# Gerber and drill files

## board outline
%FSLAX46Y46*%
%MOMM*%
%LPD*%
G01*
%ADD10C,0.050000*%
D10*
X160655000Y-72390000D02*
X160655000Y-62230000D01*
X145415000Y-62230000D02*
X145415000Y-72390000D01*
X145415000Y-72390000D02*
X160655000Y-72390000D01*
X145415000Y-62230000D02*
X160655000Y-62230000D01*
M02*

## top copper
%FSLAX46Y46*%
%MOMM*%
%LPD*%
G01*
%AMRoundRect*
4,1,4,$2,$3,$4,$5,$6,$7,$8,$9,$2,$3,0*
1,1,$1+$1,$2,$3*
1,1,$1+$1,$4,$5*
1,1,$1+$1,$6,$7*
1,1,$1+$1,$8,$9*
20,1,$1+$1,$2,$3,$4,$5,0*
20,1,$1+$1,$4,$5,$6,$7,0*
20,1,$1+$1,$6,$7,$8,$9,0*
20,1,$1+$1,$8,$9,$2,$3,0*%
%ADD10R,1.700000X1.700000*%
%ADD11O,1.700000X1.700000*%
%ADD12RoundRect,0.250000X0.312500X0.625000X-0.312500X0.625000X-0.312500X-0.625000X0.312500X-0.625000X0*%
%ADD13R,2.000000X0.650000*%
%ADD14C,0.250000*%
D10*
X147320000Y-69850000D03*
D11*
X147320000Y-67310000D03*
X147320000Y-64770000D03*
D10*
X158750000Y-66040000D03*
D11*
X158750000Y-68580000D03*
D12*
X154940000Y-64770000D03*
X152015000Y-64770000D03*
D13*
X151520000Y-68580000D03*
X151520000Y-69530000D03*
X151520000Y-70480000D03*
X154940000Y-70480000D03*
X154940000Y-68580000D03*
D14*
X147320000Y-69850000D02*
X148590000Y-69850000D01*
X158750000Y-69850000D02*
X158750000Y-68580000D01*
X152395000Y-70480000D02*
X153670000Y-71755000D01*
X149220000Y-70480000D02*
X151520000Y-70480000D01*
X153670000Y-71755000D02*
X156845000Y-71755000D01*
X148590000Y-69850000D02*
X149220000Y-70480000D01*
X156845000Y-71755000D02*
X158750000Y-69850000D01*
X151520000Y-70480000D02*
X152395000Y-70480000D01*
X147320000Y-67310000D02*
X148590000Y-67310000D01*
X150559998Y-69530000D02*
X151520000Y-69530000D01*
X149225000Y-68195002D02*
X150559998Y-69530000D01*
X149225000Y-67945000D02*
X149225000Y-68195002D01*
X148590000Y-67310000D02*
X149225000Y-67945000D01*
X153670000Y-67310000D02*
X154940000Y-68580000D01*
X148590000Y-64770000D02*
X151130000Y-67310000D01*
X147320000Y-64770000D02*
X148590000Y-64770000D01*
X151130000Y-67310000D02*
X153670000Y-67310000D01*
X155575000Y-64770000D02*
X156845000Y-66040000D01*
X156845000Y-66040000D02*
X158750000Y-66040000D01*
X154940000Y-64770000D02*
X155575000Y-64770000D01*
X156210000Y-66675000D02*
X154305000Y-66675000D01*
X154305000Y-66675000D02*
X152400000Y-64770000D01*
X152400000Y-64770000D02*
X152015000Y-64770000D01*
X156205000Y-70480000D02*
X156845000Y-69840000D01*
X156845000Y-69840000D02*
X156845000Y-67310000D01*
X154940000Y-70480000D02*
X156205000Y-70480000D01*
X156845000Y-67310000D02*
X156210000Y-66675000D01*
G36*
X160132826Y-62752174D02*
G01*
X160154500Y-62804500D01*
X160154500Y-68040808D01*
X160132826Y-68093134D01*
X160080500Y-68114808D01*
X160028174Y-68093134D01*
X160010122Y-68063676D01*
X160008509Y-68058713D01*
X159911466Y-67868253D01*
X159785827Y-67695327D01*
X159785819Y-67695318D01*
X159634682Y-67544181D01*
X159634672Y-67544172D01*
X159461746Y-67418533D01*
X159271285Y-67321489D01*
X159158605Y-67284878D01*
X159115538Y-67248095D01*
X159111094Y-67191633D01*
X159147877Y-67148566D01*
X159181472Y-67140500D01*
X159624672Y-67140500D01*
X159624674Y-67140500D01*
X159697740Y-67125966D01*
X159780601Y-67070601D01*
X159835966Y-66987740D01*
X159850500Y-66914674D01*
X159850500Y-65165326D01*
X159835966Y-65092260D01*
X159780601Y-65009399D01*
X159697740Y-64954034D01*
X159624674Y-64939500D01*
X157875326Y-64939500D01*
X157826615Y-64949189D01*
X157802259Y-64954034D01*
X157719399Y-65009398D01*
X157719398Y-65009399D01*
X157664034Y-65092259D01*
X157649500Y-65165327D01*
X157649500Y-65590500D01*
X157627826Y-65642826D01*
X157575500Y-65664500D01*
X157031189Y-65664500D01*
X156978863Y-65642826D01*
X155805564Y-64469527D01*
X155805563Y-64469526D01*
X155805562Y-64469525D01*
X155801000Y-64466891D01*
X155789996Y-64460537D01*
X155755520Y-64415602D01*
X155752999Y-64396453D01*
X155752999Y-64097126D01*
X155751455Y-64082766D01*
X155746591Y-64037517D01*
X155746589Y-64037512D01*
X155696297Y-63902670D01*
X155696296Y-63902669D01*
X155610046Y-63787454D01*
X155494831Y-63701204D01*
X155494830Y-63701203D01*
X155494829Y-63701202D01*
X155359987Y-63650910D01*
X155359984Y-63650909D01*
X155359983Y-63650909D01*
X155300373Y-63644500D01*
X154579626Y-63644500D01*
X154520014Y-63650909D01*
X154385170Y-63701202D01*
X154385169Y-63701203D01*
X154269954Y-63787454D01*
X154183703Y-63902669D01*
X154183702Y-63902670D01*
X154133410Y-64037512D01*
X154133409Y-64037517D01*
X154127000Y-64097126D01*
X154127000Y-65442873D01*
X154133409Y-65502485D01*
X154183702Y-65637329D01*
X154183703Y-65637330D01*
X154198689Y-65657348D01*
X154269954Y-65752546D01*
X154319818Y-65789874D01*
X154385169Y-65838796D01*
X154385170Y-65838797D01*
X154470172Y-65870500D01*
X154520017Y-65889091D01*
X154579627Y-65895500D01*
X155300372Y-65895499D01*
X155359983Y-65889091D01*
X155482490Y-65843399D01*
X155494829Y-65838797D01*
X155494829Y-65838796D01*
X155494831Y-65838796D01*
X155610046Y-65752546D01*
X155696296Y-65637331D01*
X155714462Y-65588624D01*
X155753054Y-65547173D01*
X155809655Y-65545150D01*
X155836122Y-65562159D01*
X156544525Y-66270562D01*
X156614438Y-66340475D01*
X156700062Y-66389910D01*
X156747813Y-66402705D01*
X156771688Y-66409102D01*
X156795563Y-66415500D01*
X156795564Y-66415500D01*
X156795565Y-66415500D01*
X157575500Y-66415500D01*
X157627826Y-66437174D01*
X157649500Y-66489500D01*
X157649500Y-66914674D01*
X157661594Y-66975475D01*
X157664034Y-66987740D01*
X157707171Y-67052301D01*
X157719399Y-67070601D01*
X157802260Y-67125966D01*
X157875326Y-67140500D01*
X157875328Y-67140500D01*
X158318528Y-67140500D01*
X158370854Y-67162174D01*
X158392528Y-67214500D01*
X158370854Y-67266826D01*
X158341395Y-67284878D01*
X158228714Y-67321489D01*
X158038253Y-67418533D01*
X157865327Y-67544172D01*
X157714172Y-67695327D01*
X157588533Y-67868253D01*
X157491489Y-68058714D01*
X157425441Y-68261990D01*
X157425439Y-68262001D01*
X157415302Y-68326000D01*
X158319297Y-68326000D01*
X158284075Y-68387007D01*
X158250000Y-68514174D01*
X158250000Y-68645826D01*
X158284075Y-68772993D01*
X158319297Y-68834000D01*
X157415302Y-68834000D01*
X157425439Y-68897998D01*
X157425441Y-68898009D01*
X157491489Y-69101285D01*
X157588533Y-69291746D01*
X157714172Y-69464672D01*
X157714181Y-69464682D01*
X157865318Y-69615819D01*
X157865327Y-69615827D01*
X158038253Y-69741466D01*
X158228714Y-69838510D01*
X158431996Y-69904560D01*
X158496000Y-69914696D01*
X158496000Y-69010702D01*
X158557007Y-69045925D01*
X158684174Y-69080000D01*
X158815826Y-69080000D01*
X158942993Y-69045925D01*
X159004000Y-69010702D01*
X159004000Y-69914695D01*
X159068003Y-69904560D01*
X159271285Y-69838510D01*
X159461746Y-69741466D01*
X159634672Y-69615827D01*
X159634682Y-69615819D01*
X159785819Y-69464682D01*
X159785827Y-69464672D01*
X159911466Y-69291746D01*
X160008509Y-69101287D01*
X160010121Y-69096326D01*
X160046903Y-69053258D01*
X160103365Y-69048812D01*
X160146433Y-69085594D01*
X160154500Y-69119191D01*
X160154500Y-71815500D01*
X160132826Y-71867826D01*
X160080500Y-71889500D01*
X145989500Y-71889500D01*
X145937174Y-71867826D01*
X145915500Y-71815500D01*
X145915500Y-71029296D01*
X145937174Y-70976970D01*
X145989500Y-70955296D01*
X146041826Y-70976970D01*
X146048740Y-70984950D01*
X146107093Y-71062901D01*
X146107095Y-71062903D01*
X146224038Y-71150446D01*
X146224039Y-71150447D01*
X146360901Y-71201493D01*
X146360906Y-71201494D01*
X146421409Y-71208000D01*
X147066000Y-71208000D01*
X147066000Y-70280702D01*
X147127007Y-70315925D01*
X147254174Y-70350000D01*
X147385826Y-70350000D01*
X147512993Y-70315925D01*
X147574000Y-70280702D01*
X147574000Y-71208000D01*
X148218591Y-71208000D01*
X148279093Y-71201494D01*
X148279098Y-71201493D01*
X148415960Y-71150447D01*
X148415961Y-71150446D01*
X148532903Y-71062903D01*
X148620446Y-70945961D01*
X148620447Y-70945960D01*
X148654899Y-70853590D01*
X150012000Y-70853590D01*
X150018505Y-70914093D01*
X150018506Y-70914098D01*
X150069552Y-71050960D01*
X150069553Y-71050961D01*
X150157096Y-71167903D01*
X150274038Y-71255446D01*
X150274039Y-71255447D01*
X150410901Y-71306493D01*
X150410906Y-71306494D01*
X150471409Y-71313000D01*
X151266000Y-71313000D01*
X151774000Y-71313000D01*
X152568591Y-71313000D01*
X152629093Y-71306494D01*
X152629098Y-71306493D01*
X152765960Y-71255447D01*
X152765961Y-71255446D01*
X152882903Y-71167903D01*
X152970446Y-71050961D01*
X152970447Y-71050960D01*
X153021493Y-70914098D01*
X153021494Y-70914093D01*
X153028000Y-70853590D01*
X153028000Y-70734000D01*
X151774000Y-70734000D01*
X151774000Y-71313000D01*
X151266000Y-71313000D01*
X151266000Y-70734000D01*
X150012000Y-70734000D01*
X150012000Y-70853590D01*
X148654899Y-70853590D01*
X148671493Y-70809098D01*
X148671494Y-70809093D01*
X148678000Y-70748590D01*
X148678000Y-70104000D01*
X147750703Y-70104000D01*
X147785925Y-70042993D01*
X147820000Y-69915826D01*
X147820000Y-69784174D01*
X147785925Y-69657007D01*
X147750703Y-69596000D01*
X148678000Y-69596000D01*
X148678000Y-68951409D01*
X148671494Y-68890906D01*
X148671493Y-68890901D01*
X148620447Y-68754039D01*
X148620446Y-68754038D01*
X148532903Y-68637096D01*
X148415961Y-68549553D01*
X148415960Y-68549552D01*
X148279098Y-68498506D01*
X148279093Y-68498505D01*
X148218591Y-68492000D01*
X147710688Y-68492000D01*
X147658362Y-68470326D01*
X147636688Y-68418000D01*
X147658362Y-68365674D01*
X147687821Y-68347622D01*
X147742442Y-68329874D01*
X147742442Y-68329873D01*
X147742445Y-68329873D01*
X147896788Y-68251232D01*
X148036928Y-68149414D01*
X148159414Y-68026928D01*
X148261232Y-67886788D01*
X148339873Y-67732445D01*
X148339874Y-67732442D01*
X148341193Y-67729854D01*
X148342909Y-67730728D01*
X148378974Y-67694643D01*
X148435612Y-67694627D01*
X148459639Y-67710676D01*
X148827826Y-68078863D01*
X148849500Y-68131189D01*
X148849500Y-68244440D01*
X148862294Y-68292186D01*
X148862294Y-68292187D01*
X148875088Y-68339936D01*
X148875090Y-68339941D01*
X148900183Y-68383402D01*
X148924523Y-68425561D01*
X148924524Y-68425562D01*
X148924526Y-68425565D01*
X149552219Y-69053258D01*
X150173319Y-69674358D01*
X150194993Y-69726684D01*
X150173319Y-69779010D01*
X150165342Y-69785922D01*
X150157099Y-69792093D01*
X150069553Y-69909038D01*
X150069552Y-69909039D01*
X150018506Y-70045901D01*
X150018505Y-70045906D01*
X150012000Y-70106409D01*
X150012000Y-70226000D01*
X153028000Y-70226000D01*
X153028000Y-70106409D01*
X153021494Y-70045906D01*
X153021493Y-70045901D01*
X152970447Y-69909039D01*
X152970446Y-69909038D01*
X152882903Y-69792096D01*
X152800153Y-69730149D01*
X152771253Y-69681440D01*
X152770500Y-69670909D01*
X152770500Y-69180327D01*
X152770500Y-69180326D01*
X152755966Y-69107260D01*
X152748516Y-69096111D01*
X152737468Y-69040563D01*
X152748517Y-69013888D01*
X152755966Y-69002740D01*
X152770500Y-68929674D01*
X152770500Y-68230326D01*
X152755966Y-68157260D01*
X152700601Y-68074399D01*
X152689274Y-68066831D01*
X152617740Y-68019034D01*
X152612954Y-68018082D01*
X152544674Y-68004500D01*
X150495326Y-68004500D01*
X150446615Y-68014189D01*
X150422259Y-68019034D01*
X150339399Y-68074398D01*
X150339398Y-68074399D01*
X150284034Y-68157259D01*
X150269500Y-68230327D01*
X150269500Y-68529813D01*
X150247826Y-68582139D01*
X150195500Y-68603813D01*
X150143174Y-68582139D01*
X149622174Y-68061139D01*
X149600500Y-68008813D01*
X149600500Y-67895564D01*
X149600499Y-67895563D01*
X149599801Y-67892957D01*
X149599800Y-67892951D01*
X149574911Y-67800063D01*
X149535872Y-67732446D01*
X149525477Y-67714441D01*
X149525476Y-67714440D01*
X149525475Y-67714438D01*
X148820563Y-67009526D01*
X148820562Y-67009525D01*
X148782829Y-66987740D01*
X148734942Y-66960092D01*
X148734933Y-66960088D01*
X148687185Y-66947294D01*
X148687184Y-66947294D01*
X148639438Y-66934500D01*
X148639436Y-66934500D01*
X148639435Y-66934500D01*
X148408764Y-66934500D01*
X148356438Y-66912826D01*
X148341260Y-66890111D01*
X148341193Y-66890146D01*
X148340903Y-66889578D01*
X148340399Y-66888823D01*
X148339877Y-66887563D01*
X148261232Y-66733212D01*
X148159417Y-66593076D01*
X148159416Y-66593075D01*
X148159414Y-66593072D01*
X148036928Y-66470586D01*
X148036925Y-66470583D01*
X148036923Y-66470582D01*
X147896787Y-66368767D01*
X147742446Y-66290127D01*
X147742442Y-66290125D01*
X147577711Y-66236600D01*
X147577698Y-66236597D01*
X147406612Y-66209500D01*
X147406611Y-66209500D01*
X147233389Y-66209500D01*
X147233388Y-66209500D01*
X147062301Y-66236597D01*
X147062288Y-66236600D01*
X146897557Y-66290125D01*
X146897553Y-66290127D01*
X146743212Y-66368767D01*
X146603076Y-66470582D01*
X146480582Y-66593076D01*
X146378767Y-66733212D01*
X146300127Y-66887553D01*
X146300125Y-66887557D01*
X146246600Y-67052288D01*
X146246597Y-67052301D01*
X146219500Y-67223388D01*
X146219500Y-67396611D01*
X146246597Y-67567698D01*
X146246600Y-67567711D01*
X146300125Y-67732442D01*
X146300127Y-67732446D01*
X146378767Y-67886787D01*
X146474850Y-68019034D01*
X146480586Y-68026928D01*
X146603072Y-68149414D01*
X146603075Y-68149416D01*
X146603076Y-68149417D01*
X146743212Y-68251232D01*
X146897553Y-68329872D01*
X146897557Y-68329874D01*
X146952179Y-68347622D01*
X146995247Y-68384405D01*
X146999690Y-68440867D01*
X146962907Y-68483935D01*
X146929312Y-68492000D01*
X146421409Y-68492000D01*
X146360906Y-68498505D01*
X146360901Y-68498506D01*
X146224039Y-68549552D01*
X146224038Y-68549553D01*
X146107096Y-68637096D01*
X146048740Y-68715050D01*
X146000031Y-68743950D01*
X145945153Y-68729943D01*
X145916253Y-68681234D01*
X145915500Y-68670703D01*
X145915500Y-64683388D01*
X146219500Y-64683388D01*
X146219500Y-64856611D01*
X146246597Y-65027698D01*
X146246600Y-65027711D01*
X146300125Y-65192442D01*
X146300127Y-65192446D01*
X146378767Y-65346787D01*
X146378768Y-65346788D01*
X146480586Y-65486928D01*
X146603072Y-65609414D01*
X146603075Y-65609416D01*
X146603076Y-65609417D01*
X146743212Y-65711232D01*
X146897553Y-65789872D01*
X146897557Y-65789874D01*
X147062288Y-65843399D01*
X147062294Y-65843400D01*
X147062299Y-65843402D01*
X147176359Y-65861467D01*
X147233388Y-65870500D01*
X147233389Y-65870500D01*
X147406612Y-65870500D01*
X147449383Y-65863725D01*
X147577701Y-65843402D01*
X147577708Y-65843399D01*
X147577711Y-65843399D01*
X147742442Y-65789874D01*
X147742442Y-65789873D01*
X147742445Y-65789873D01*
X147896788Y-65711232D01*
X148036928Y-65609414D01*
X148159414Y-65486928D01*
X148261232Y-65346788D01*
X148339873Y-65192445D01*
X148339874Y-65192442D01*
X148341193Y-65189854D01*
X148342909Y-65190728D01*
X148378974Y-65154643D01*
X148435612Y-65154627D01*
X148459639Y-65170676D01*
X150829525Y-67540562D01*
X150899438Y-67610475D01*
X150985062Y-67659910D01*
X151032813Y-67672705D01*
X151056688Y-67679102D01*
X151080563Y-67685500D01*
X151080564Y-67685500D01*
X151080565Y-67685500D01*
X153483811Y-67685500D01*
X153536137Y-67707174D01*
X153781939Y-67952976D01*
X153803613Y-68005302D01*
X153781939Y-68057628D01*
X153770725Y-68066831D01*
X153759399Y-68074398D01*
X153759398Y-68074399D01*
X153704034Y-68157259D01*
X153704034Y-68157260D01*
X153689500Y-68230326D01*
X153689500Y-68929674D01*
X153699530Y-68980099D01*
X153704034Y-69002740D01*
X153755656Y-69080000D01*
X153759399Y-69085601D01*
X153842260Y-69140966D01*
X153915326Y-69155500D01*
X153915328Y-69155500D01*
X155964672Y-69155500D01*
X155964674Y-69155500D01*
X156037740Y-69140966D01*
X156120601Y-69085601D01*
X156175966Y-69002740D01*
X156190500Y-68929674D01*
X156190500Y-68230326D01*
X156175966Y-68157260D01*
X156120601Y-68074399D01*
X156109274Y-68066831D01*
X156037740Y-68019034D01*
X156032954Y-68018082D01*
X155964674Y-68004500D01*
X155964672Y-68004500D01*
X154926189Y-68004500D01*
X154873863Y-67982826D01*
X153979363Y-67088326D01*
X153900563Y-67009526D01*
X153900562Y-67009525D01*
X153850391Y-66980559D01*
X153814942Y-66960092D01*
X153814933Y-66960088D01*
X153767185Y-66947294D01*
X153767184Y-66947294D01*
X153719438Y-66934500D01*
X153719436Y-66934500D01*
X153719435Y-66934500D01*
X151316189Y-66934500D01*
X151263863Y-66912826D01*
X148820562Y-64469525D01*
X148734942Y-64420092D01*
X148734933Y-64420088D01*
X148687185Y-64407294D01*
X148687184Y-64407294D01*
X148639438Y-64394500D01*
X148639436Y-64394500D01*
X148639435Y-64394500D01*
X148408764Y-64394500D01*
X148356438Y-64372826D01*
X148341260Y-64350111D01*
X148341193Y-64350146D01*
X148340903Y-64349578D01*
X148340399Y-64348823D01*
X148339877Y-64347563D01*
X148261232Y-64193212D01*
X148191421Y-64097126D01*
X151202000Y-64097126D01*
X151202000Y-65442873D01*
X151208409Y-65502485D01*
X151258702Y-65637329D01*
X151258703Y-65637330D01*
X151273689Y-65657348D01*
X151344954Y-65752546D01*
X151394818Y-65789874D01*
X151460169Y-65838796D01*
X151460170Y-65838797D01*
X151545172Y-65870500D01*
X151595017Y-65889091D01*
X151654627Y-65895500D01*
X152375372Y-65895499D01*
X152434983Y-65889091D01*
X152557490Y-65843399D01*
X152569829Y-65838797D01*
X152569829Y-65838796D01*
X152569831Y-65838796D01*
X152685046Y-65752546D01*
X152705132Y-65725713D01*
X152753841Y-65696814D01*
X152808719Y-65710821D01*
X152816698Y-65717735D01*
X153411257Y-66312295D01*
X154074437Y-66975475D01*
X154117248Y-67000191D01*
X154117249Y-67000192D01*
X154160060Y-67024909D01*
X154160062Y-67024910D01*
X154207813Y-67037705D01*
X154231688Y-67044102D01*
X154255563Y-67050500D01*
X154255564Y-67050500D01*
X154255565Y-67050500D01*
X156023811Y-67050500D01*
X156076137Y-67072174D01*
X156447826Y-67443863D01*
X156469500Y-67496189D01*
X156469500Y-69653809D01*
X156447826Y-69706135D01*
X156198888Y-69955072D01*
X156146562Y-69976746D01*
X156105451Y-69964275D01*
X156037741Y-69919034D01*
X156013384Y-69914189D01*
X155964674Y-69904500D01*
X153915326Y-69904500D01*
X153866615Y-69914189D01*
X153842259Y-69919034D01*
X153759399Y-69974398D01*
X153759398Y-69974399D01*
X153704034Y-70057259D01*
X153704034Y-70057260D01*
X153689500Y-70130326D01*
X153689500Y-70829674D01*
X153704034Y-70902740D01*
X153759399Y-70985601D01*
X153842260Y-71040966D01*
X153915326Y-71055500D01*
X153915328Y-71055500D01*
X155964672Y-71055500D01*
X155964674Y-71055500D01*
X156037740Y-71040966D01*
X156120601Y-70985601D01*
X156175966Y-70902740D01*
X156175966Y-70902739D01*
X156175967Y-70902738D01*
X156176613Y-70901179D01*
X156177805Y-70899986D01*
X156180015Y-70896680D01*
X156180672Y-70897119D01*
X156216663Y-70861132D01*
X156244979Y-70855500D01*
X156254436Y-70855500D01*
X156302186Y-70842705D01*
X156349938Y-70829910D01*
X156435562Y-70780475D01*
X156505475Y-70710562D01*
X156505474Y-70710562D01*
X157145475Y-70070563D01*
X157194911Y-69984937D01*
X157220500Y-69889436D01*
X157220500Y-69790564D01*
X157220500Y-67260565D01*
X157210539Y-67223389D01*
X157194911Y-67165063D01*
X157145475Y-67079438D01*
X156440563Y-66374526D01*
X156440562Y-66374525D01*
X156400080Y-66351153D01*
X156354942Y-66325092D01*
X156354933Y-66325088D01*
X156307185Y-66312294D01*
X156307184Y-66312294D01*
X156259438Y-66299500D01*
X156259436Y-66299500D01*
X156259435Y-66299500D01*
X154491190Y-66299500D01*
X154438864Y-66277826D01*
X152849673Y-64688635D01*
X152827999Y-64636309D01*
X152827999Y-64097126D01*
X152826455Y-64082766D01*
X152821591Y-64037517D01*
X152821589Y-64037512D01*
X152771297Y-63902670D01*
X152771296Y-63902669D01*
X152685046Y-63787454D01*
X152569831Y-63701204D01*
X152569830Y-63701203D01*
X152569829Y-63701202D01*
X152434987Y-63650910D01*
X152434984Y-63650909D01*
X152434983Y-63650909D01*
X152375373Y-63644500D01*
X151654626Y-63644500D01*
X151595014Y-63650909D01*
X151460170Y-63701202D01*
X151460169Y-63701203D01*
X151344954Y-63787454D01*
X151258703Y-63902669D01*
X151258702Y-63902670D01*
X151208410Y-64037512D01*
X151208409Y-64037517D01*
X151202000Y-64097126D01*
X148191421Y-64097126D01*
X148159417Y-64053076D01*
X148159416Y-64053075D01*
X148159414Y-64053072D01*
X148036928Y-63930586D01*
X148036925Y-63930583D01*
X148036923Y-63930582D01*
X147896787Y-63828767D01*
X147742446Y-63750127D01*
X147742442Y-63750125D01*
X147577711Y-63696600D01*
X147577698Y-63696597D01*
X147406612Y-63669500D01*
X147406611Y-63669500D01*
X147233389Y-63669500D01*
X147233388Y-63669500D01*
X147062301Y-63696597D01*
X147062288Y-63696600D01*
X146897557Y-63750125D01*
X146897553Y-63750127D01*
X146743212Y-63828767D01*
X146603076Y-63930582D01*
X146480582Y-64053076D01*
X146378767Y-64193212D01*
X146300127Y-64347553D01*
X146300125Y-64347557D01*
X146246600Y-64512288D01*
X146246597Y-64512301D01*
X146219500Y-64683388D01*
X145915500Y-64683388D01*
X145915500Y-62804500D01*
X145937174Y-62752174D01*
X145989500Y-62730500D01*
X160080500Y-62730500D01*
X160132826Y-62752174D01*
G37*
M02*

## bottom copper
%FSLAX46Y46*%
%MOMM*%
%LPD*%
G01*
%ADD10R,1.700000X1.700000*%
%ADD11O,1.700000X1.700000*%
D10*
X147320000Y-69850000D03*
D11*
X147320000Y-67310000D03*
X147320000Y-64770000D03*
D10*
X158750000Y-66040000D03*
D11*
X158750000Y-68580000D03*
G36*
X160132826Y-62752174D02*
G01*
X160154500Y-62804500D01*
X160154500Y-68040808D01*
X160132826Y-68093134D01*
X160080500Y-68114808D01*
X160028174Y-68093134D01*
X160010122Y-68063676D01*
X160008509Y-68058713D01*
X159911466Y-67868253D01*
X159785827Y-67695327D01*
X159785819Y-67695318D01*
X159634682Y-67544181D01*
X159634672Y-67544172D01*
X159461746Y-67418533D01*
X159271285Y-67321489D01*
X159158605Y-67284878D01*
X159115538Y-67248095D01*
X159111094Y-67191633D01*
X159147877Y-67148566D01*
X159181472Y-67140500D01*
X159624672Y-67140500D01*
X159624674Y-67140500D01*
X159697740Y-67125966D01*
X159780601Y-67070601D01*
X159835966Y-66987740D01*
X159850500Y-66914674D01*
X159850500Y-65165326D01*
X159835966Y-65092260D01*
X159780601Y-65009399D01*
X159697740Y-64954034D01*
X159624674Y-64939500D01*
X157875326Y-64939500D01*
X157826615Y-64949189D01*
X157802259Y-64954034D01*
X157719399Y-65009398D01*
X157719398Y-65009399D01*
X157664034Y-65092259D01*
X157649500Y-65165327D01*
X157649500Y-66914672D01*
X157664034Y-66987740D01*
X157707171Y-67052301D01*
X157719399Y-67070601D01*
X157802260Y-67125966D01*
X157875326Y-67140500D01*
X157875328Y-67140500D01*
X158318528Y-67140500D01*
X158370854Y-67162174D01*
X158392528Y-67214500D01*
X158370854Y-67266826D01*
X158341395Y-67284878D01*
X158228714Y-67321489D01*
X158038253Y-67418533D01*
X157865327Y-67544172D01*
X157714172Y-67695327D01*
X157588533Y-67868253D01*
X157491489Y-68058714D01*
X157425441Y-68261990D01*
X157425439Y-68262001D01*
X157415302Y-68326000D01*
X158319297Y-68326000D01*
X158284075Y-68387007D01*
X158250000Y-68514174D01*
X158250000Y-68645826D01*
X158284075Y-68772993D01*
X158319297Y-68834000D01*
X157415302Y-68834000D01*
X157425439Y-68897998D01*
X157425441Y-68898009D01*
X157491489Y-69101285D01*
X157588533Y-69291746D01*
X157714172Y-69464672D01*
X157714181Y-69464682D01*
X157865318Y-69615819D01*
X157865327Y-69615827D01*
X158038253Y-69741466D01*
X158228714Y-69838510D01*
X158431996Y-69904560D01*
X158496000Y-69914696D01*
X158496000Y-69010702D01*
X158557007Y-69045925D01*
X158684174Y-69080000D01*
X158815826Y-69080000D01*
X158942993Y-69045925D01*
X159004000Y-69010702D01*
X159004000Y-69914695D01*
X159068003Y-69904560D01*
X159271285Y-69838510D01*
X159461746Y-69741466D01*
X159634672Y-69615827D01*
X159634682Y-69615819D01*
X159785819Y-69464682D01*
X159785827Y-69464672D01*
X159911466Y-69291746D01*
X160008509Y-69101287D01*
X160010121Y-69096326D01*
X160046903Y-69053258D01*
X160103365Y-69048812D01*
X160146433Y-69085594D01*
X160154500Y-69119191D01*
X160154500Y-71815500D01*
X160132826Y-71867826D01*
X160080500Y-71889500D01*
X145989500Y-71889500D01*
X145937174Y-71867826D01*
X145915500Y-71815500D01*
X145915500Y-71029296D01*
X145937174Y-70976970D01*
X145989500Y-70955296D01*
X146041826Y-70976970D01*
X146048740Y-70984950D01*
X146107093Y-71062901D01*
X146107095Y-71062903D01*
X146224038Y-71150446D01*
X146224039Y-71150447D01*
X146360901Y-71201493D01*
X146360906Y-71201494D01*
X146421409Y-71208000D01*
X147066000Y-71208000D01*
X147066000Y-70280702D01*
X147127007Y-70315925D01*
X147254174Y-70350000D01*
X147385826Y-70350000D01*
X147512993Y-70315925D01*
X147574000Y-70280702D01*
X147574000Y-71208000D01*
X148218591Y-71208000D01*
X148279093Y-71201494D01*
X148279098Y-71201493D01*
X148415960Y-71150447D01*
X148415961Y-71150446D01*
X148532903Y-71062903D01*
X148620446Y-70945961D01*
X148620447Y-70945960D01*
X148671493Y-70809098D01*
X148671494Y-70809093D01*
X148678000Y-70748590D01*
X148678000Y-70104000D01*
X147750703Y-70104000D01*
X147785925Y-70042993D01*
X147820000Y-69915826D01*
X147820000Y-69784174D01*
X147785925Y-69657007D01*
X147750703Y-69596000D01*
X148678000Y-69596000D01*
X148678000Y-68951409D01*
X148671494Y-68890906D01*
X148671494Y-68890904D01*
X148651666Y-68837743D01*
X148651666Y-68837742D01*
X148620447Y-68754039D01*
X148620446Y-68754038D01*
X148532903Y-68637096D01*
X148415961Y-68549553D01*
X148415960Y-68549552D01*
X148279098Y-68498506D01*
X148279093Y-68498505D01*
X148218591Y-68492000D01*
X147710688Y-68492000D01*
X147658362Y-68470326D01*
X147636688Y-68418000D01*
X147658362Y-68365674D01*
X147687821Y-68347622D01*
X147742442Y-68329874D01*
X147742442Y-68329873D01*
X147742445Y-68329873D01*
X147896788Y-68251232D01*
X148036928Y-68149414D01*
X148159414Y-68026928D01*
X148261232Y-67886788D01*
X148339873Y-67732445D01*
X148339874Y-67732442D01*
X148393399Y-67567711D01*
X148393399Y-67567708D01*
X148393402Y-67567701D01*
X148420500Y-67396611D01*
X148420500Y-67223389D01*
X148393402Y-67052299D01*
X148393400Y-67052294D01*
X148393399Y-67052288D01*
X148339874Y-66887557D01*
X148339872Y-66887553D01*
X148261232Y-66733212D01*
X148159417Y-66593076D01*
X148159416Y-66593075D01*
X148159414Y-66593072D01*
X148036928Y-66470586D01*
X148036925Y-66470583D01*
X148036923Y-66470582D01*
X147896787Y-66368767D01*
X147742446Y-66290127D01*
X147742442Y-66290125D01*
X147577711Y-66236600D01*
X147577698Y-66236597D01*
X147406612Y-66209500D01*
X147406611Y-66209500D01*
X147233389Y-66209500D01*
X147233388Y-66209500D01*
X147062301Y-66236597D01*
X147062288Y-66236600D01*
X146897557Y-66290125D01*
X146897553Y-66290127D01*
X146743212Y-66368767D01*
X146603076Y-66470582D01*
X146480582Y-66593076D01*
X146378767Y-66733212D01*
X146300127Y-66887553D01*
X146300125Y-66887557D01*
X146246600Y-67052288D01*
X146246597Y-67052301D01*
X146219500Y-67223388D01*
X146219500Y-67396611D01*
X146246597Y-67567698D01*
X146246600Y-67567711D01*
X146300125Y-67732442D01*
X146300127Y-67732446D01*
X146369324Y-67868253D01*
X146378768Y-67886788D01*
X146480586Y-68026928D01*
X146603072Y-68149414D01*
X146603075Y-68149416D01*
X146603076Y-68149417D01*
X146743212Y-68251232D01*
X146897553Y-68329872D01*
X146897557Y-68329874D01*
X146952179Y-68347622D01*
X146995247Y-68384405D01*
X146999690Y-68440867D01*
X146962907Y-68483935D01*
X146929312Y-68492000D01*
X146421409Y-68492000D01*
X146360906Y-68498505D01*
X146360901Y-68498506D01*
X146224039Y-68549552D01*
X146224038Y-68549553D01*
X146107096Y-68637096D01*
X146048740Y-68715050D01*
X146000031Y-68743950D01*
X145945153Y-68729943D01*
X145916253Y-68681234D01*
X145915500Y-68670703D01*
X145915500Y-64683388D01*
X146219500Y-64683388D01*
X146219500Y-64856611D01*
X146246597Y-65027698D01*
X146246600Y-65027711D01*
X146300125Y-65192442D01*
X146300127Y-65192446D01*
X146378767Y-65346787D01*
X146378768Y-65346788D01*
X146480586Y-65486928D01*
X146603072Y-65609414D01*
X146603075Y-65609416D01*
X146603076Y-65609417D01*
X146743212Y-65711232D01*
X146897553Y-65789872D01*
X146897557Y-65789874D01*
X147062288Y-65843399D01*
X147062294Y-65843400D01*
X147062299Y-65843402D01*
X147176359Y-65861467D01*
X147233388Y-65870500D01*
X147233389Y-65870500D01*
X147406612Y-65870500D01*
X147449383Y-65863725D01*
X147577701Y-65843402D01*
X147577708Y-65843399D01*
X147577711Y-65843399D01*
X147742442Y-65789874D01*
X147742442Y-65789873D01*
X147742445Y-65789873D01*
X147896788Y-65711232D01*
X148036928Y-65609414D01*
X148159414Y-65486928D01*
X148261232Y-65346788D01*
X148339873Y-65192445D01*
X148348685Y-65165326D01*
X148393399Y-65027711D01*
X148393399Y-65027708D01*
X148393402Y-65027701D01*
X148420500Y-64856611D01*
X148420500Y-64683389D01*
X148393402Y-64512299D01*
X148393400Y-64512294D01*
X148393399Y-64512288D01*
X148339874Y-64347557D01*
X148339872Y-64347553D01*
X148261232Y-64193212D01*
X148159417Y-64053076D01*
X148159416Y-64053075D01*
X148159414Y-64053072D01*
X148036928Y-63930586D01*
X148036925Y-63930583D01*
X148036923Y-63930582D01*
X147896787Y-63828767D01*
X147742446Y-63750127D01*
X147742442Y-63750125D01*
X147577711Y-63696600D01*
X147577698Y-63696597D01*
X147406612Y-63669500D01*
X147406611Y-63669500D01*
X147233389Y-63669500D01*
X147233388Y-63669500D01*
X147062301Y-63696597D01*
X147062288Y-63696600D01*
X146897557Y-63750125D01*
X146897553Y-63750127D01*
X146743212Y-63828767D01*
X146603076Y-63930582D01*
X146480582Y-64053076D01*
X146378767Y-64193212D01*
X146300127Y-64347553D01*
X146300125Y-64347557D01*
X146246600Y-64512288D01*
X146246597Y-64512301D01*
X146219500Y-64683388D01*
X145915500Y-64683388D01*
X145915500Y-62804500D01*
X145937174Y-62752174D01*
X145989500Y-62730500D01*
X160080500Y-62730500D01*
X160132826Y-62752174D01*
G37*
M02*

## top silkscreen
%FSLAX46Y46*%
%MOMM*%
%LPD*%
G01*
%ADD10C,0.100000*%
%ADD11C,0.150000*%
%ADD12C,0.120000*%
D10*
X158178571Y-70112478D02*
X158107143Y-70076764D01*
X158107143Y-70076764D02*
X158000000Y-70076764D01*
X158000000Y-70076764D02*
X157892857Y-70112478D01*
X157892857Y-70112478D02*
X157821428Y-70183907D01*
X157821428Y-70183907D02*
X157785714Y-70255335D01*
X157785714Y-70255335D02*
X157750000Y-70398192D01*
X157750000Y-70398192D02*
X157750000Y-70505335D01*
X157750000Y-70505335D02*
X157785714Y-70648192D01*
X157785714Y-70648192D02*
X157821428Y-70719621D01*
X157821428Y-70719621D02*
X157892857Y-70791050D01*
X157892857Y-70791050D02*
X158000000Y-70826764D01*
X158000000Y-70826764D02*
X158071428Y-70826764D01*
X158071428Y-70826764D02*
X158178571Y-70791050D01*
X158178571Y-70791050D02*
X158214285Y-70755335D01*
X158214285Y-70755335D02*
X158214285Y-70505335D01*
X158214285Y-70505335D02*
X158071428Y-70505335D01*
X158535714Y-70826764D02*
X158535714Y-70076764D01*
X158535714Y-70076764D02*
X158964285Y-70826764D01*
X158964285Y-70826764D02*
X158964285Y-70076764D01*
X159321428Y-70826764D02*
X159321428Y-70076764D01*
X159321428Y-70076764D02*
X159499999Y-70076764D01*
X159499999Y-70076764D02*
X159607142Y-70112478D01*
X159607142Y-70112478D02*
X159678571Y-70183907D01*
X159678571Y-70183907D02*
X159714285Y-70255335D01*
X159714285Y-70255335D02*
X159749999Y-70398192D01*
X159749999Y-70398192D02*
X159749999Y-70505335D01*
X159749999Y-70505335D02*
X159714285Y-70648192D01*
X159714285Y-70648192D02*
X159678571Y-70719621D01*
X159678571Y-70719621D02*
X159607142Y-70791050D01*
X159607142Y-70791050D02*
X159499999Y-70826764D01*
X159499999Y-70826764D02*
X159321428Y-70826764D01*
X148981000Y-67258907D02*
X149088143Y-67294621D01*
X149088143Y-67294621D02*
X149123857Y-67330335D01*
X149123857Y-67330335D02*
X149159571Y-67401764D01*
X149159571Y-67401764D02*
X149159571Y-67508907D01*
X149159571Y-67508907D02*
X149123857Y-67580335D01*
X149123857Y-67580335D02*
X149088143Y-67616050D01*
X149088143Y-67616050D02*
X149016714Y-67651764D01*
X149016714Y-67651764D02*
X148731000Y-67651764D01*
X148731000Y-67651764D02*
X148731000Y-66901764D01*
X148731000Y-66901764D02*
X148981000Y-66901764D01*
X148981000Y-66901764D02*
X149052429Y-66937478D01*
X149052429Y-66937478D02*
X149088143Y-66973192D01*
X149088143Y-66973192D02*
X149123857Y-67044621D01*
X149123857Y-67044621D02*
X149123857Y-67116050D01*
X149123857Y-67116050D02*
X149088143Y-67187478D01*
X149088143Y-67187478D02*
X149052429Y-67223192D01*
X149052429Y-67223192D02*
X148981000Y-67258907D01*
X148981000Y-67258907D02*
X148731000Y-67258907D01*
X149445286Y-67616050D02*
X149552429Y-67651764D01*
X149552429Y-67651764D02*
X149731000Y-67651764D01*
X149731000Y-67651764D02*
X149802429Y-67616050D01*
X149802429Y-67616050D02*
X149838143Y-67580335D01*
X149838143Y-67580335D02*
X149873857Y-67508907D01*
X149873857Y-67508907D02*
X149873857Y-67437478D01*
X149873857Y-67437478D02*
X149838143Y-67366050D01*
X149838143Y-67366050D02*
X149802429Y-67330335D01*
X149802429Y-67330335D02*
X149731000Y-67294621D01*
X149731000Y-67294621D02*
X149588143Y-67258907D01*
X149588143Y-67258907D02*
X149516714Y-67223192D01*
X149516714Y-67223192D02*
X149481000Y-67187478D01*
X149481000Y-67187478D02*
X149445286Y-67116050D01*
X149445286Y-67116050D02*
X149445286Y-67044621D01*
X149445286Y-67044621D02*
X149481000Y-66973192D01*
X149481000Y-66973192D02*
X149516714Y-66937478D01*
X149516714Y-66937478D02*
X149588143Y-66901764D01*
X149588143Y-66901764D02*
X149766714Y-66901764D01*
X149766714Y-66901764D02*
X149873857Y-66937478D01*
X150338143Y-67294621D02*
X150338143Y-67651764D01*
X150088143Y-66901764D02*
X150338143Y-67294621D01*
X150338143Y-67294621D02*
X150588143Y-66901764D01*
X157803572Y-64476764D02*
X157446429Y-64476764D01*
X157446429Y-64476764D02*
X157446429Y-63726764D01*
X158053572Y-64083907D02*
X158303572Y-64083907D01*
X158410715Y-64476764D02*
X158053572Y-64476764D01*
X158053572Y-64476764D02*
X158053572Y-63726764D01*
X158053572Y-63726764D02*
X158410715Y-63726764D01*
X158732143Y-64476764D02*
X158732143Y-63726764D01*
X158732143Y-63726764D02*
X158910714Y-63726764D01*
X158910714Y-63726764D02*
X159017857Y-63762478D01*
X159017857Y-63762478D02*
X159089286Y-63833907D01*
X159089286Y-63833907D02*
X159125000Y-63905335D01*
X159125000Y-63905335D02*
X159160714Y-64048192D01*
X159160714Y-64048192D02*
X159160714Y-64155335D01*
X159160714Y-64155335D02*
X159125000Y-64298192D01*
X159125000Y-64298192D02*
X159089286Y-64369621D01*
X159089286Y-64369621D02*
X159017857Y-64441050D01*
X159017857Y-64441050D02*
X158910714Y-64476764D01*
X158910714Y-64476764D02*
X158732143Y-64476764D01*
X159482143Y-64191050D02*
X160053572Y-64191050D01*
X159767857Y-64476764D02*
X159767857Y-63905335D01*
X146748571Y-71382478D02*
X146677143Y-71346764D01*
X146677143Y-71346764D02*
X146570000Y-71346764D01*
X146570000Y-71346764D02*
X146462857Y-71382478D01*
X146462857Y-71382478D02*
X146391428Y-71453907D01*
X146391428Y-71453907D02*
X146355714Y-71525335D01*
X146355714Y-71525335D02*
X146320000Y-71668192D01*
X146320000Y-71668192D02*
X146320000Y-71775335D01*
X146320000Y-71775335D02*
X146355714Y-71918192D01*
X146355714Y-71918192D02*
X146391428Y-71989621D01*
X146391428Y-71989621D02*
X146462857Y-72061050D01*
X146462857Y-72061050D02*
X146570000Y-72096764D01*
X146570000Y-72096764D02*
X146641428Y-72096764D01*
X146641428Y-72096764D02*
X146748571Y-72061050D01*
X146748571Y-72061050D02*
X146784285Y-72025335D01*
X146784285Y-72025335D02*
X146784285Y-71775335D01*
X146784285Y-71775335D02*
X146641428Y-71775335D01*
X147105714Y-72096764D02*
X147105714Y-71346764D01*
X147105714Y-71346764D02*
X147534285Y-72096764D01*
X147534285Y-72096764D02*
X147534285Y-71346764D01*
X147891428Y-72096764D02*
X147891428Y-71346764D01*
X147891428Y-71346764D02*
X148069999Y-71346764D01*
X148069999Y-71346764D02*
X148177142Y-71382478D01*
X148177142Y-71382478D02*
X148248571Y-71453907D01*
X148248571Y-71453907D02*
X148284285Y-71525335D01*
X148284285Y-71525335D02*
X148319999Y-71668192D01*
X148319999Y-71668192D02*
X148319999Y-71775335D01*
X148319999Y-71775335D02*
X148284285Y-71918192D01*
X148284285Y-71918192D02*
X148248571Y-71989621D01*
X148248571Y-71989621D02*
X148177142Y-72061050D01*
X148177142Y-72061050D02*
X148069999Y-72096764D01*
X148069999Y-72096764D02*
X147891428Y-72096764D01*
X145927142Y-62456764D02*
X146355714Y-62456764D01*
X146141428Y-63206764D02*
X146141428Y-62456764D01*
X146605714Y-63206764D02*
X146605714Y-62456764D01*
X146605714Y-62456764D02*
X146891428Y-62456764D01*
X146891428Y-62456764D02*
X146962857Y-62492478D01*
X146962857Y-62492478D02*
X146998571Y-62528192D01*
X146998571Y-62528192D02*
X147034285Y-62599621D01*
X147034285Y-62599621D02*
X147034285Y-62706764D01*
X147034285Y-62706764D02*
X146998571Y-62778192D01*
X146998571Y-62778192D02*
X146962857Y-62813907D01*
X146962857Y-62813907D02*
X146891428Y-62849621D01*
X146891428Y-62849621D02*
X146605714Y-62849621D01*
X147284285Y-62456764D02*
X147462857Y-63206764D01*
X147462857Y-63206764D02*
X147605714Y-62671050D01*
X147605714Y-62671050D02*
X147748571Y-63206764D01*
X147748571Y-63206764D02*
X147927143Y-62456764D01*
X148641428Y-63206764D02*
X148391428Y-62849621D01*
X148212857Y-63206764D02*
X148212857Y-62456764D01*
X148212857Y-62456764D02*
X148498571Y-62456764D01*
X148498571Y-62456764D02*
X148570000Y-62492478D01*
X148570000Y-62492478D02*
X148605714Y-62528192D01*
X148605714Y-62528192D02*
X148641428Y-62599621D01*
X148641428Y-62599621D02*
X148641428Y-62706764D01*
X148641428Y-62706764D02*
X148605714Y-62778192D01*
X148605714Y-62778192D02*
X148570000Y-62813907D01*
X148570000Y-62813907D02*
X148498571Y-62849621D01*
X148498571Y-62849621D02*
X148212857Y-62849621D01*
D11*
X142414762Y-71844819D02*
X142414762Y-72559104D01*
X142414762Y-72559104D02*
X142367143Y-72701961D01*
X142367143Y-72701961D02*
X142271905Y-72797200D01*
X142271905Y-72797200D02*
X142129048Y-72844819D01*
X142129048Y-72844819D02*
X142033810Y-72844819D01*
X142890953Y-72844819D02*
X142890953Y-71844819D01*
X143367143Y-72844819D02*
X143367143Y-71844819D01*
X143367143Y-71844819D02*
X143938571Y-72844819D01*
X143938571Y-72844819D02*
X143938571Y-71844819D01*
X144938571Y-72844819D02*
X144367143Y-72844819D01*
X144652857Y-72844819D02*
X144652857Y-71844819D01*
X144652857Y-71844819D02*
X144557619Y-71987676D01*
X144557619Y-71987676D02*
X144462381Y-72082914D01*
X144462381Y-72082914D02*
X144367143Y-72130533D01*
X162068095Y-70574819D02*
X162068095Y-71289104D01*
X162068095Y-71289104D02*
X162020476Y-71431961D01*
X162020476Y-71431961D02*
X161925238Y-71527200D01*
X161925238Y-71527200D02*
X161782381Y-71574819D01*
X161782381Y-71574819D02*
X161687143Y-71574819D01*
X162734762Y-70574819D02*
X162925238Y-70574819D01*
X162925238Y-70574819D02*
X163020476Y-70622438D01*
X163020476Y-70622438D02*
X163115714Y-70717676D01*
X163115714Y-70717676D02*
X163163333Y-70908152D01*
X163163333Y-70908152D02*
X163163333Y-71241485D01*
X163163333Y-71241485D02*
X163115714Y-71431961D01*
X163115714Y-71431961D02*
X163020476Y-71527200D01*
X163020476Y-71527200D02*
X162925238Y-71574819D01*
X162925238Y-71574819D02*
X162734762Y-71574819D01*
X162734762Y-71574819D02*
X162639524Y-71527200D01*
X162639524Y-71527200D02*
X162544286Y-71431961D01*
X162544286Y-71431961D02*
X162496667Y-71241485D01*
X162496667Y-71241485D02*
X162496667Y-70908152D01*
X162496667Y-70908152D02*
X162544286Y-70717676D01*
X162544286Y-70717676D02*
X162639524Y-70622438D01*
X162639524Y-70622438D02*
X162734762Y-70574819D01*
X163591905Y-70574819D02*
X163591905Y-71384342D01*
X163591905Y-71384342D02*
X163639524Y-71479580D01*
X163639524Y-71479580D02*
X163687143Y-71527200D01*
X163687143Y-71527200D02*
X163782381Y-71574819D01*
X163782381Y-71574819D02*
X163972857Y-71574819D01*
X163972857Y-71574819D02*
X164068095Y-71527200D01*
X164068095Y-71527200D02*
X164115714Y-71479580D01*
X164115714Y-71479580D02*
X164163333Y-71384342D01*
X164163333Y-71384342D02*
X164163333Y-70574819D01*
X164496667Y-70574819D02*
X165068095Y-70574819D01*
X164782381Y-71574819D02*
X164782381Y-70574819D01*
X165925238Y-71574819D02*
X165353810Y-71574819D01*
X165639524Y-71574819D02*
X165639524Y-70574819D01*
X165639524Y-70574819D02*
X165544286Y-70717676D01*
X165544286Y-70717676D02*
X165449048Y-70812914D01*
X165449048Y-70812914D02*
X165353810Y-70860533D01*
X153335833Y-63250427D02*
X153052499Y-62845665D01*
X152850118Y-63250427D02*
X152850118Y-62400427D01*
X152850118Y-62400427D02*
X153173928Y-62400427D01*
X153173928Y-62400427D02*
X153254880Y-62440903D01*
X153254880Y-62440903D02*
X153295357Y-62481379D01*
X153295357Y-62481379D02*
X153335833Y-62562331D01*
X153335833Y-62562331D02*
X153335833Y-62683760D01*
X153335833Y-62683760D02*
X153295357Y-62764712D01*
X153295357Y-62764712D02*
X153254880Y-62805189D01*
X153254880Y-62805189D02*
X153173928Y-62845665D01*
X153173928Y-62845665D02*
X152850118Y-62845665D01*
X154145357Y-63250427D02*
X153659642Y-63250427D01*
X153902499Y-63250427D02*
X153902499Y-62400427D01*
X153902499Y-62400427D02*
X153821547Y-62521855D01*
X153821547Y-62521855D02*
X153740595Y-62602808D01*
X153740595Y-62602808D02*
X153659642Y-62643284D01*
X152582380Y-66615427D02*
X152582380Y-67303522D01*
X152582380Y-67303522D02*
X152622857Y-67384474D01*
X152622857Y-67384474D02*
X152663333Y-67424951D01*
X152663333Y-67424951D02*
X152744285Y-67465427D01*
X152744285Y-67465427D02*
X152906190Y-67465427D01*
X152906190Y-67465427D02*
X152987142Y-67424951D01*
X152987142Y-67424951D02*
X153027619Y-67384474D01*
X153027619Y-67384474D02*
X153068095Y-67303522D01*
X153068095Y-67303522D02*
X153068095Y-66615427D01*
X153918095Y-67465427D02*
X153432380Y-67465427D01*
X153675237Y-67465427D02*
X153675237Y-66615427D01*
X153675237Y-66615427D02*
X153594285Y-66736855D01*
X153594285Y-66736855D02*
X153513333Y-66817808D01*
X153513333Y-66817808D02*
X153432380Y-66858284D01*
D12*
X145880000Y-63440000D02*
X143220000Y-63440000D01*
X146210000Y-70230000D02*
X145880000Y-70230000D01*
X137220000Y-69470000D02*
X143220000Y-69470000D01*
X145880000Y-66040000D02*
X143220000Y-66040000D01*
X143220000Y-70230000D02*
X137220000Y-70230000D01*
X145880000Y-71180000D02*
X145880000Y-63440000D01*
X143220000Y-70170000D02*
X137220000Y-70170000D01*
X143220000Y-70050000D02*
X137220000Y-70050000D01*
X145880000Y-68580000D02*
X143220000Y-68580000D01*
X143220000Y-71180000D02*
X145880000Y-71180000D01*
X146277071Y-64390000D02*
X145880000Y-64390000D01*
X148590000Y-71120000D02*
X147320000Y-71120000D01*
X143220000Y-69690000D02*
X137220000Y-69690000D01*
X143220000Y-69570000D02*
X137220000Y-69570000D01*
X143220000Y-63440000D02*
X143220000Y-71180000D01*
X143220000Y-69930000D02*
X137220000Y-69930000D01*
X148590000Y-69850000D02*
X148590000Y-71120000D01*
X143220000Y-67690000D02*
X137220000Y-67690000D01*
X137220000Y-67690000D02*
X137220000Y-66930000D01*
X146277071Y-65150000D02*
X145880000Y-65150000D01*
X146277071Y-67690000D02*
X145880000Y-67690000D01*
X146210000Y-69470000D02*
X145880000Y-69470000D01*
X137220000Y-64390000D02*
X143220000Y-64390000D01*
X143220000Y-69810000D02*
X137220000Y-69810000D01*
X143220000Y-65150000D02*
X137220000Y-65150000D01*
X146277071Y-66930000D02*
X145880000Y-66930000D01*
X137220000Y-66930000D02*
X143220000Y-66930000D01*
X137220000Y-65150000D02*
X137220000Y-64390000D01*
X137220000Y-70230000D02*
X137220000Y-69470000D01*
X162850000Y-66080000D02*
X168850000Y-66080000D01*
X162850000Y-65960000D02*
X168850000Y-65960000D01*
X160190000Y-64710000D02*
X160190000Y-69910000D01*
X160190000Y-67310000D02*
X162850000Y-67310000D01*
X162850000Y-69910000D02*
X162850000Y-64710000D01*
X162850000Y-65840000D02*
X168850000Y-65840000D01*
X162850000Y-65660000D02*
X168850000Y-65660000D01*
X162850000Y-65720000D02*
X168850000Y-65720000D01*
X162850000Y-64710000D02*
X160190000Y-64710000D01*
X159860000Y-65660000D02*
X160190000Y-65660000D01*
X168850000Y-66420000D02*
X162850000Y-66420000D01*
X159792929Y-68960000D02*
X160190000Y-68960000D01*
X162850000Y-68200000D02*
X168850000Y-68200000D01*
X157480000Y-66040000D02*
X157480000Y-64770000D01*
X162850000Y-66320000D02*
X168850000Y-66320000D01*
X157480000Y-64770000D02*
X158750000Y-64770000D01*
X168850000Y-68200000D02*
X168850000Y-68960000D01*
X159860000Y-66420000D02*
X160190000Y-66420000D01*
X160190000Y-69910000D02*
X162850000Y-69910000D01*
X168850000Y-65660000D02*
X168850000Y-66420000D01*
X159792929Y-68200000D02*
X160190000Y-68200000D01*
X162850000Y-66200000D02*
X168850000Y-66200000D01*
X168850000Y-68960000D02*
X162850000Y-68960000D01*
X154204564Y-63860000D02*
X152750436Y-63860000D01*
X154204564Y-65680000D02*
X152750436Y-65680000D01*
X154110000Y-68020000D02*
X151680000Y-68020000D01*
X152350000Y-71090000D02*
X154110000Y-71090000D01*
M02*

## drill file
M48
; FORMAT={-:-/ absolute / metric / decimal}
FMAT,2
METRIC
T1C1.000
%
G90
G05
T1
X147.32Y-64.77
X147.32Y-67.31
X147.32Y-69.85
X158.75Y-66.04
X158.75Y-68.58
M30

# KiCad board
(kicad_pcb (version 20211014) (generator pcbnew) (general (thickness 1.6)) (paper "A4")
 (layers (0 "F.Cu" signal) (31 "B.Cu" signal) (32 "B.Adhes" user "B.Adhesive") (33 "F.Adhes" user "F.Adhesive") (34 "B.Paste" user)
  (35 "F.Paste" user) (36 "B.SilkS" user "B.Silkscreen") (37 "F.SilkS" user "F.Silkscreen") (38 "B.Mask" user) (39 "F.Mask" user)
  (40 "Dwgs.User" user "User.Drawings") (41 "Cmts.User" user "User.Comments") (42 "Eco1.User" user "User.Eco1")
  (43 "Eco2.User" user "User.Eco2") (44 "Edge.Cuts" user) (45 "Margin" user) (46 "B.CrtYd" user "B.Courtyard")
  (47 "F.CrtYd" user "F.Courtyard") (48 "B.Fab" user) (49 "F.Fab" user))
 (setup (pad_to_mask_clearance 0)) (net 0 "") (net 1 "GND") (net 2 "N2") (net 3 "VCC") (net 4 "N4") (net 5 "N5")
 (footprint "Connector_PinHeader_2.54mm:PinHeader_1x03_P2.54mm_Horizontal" (layer "F.Cu") (at 147.32 69.85 180)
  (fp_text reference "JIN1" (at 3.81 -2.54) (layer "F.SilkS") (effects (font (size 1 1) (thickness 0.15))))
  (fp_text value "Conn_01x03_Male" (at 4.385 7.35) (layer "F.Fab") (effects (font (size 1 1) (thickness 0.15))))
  (fp_line (start 1.44 6.41) (end 4.1 6.41) (layer "F.SilkS") (width 0.12))
  (fp_line (start 1.11 -0.38) (end 1.44 -0.38) (layer "F.SilkS") (width 0.12))
  (fp_line (start 10.1 0.38) (end 4.1 0.38) (layer "F.SilkS") (width 0.12))
  (fp_line (start 1.44 3.81) (end 4.1 3.81) (layer "F.SilkS") (width 0.12))
  (fp_line (start 4.1 -0.38) (end 10.1 -0.38) (layer "F.SilkS") (width 0.12))
  (fp_line (start 1.44 -1.33) (end 1.44 6.41) (layer "F.SilkS") (width 0.12))
  (fp_line (start 4.1 -0.32) (end 10.1 -0.32) (layer "F.SilkS") (width 0.12))
  (fp_line (start 4.1 -0.2) (end 10.1 -0.2) (layer "F.SilkS") (width 0.12))
  (fp_line (start 1.44 1.27) (end 4.1 1.27) (layer "F.SilkS") (width 0.12))
  (fp_line (start 4.1 -1.33) (end 1.44 -1.33) (layer "F.SilkS") (width 0.12))
  (fp_line (start 1.042929 5.46) (end 1.44 5.46) (layer "F.SilkS") (width 0.12))
  (fp_line (start -1.27 -1.27) (end 0 -1.27) (layer "F.SilkS") (width 0.12))
  (fp_line (start 4.1 0.16) (end 10.1 0.16) (layer "F.SilkS") (width 0.12))
  (fp_line (start 4.1 0.28) (end 10.1 0.28) (layer "F.SilkS") (width 0.12))
  (fp_line (start 4.1 6.41) (end 4.1 -1.33) (layer "F.SilkS") (width 0.12))
  (fp_line (start 4.1 -0.08) (end 10.1 -0.08) (layer "F.SilkS") (width 0.12))
  (fp_line (start -1.27 0) (end -1.27 -1.27) (layer "F.SilkS") (width 0.12))
  (fp_line (start 4.1 2.16) (end 10.1 2.16) (layer "F.SilkS") (width 0.12))
  (fp_line (start 10.1 2.16) (end 10.1 2.92) (layer "F.SilkS") (width 0.12))
  (fp_line (start 1.042929 4.7) (end 1.44 4.7) (layer "F.SilkS") (width 0.12))
  (fp_line (start 1.042929 2.16) (end 1.44 2.16) (layer "F.SilkS") (width 0.12))
  (fp_line (start 1.11 0.38) (end 1.44 0.38) (layer "F.SilkS") (width 0.12))
  (fp_line (start 10.1 5.46) (end 4.1 5.46) (layer "F.SilkS") (width 0.12))
  (fp_line (start 4.1 0.04) (end 10.1 0.04) (layer "F.SilkS") (width 0.12))
  (fp_line (start 4.1 4.7) (end 10.1 4.7) (layer "F.SilkS") (width 0.12))
  (fp_line (start 1.042929 2.92) (end 1.44 2.92) (layer "F.SilkS") (width 0.12))
  (fp_line (start 10.1 2.92) (end 4.1 2.92) (layer "F.SilkS") (width 0.12))
  (fp_line (start 10.1 4.7) (end 10.1 5.46) (layer "F.SilkS") (width 0.12))
  (fp_line (start 10.1 -0.38) (end 10.1 0.38) (layer "F.SilkS") (width 0.12))
  (pad "1" thru_hole rect locked (at 0 0 180) (size 1.7 1.7) (drill 1) (layers *.Cu *.Mask) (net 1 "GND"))
  (pad "2" thru_hole oval locked (at 0 2.54 180) (size 1.7 1.7) (drill 1) (layers *.Cu *.Mask) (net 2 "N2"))
  (pad "3" thru_hole oval locked (at 0 5.08 180) (size 1.7 1.7) (drill 1) (layers *.Cu *.Mask) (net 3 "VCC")))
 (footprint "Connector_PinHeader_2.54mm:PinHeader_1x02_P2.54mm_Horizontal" (layer "F.Cu") (at 158.75 66.04)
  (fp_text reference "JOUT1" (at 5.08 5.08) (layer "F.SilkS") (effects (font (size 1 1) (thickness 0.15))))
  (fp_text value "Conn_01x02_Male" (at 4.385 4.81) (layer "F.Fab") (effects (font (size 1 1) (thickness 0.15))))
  (fp_line (start 4.1 0.04) (end 10.1 0.04) (layer "F.SilkS") (width 0.12))
  (fp_line (start 4.1 -0.08) (end 10.1 -0.08) (layer "F.SilkS") (width 0.12))
  (fp_line (start 1.44 -1.33) (end 1.44 3.87) (layer "F.SilkS") (width 0.12))
  (fp_line (start 1.44 1.27) (end 4.1 1.27) (layer "F.SilkS") (width 0.12))
  (fp_line (start 4.1 3.87) (end 4.1 -1.33) (layer "F.SilkS") (width 0.12))
  (fp_line (start 4.1 -0.2) (end 10.1 -0.2) (layer "F.SilkS") (width 0.12))
  (fp_line (start 4.1 -0.38) (end 10.1 -0.38) (layer "F.SilkS") (width 0.12))
  (fp_line (start 4.1 -0.32) (end 10.1 -0.32) (layer "F.SilkS") (width 0.12))
  (fp_line (start 4.1 -1.33) (end 1.44 -1.33) (layer "F.SilkS") (width 0.12))
  (fp_line (start 1.11 -0.38) (end 1.44 -0.38) (layer "F.SilkS") (width 0.12))
  (fp_line (start 10.1 0.38) (end 4.1 0.38) (layer "F.SilkS") (width 0.12))
  (fp_line (start 1.042929 2.92) (end 1.44 2.92) (layer "F.SilkS") (width 0.12))
  (fp_line (start 4.1 2.16) (end 10.1 2.16) (layer "F.SilkS") (width 0.12))
  (fp_line (start -1.27 0) (end -1.27 -1.27) (layer "F.SilkS") (width 0.12))
  (fp_line (start 4.1 0.28) (end 10.1 0.28) (layer "F.SilkS") (width 0.12))
  (fp_line (start -1.27 -1.27) (end 0 -1.27) (layer "F.SilkS") (width 0.12))
  (fp_line (start 10.1 2.16) (end 10.1 2.92) (layer "F.SilkS") (width 0.12))
  (fp_line (start 1.11 0.38) (end 1.44 0.38) (layer "F.SilkS") (width 0.12))
  (fp_line (start 1.44 3.87) (end 4.1 3.87) (layer "F.SilkS") (width 0.12))
  (fp_line (start 10.1 -0.38) (end 10.1 0.38) (layer "F.SilkS") (width 0.12))
  (fp_line (start 1.042929 2.16) (end 1.44 2.16) (layer "F.SilkS") (width 0.12))
  (fp_line (start 4.1 0.16) (end 10.1 0.16) (layer "F.SilkS") (width 0.12))
  (fp_line (start 10.1 2.92) (end 4.1 2.92) (layer "F.SilkS") (width 0.12))
  (pad "1" thru_hole rect locked (at 0 0) (size 1.7 1.7) (drill 1) (layers *.Cu *.Mask) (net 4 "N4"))
  (pad "2" thru_hole oval locked (at 0 2.54) (size 1.7 1.7) (drill 1) (layers *.Cu *.Mask) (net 1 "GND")))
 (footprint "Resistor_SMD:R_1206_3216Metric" (layer "F.Cu") (at 153.4775 64.77 180)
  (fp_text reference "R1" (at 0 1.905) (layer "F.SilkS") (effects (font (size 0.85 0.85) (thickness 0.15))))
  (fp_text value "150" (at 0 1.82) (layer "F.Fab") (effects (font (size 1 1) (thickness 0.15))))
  (fp_line (start -0.727064 0.91) (end 0.727064 0.91) (layer "F.SilkS") (width 0.12))
  (fp_line (start -0.727064 -0.91) (end 0.727064 -0.91) (layer "F.SilkS") (width 0.12))
  (pad "1" smd roundrect locked (at -1.4625 0 180) (size 1.125 1.75) (layers "F.Cu" "F.Paste" "F.Mask") (roundrect_rratio 0.222222)
   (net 4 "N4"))
  (pad "2" smd roundrect locked (at 1.4625 0 180) (size 1.125 1.75) (layers "F.Cu" "F.Paste" "F.Mask") (roundrect_rratio 0.222222)
   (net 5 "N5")))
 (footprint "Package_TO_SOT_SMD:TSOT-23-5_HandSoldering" (layer "F.Cu") (at 153.23 69.53)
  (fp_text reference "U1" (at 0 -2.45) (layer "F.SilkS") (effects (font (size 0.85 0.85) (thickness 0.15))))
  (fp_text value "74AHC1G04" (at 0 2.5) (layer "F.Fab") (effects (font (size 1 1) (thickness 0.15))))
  (fp_line (start 0.88 -1.51) (end -1.55 -1.51) (layer "F.SilkS") (width 0.12))
  (fp_line (start -0.88 1.56) (end 0.88 1.56) (layer "F.SilkS") (width 0.12))
  (pad "1" smd rect locked (at -1.71 -0.95) (size 2 0.65) (layers "F.Cu" "F.Paste" "F.Mask"))
  (pad "2" smd rect locked (at -1.71 0) (size 2 0.65) (layers "F.Cu" "F.Paste" "F.Mask") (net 2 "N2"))
  (pad "3" smd rect locked (at -1.71 0.95) (size 2 0.65) (layers "F.Cu" "F.Paste" "F.Mask") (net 1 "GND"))
  (pad "4" smd rect locked (at 1.71 0.95) (size 2 0.65) (layers "F.Cu" "F.Paste" "F.Mask") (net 5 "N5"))
  (pad "5" smd rect locked (at 1.71 -0.95) (size 2 0.65) (layers "F.Cu" "F.Paste" "F.Mask") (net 3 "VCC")))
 (gr_line (start 160.655 72.39) (end 160.655 62.23) (layer "Edge.Cuts") (width 0.05))
 (gr_line (start 145.415 62.23) (end 145.415 72.39) (layer "Edge.Cuts") (width 0.05))
 (gr_line (start 145.415 72.39) (end 160.655 72.39) (layer "Edge.Cuts") (width 0.05))
 (gr_line (start 145.415 62.23) (end 160.655 62.23) (layer "Edge.Cuts") (width 0.05))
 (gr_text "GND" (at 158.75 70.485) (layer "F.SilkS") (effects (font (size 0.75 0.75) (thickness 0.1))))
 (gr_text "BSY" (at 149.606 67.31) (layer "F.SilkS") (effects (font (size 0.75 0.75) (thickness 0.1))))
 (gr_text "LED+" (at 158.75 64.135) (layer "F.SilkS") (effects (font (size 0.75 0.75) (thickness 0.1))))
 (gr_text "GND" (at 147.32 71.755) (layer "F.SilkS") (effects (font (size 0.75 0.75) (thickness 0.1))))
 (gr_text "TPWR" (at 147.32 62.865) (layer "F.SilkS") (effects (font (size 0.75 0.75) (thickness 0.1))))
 (segment (start 147.32 69.85) (end 148.59 69.85) (width 0.25) (layer "F.Cu") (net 1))
 (segment (start 158.75 69.85) (end 158.75 68.58) (width 0.25) (layer "F.Cu") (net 1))
 (segment (start 152.395 70.48) (end 153.67 71.755) (width 0.25) (layer "F.Cu") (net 1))
 (segment (start 149.22 70.48) (end 151.52 70.48) (width 0.25) (layer "F.Cu") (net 1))
 (segment (start 153.67 71.755) (end 156.845 71.755) (width 0.25) (layer "F.Cu") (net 1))
 (segment (start 148.59 69.85) (end 149.22 70.48) (width 0.25) (layer "F.Cu") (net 1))
 (segment (start 156.845 71.755) (end 158.75 69.85) (width 0.25) (layer "F.Cu") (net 1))
 (segment (start 151.52 70.48) (end 152.395 70.48) (width 0.25) (layer "F.Cu") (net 1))
 (segment (start 147.32 67.31) (end 148.59 67.31) (width 0.25) (layer "F.Cu") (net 2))
 (segment (start 150.559998 69.53) (end 151.52 69.53) (width 0.25) (layer "F.Cu") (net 2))
 (segment (start 149.225 68.195002) (end 150.559998 69.53) (width 0.25) (layer "F.Cu") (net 2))
 (segment (start 149.225 67.945) (end 149.225 68.195002) (width 0.25) (layer "F.Cu") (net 2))
 (segment (start 148.59 67.31) (end 149.225 67.945) (width 0.25) (layer "F.Cu") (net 2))
 (segment (start 153.67 67.31) (end 154.94 68.58) (width 0.25) (layer "F.Cu") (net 3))
 (segment (start 148.59 64.77) (end 151.13 67.31) (width 0.25) (layer "F.Cu") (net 3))
 (segment (start 147.32 64.77) (end 148.59 64.77) (width 0.25) (layer "F.Cu") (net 3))
 (segment (start 151.13 67.31) (end 153.67 67.31) (width 0.25) (layer "F.Cu") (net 3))
 (segment (start 155.575 64.77) (end 156.845 66.04) (width 0.25) (layer "F.Cu") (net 4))
 (segment (start 156.845 66.04) (end 158.75 66.04) (width 0.25) (layer "F.Cu") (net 4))
 (segment (start 154.94 64.77) (end 155.575 64.77) (width 0.25) (layer "F.Cu") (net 4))
 (segment (start 156.21 66.675) (end 154.305 66.675) (width 0.25) (layer "F.Cu") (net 5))
 (segment (start 154.305 66.675) (end 152.4 64.77) (width 0.25) (layer "F.Cu") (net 5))
 (segment (start 152.4 64.77) (end 152.015 64.77) (width 0.25) (layer "F.Cu") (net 5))
 (segment (start 156.205 70.48) (end 156.845 69.84) (width 0.25) (layer "F.Cu") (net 5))
 (segment (start 156.845 69.84) (end 156.845 67.31) (width 0.25) (layer "F.Cu") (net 5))
 (segment (start 154.94 70.48) (end 156.205 70.48) (width 0.25) (layer "F.Cu") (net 5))
 (segment (start 156.845 67.31) (end 156.21 66.675) (width 0.25) (layer "F.Cu") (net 5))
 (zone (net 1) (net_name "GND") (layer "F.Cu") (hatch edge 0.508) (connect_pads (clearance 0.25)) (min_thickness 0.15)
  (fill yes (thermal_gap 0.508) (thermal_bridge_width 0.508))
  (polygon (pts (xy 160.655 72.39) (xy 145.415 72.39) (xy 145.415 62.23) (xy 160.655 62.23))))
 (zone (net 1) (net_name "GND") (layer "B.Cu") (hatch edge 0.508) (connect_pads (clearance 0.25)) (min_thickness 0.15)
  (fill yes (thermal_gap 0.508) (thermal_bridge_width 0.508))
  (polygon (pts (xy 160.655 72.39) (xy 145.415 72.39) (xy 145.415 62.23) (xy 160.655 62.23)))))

